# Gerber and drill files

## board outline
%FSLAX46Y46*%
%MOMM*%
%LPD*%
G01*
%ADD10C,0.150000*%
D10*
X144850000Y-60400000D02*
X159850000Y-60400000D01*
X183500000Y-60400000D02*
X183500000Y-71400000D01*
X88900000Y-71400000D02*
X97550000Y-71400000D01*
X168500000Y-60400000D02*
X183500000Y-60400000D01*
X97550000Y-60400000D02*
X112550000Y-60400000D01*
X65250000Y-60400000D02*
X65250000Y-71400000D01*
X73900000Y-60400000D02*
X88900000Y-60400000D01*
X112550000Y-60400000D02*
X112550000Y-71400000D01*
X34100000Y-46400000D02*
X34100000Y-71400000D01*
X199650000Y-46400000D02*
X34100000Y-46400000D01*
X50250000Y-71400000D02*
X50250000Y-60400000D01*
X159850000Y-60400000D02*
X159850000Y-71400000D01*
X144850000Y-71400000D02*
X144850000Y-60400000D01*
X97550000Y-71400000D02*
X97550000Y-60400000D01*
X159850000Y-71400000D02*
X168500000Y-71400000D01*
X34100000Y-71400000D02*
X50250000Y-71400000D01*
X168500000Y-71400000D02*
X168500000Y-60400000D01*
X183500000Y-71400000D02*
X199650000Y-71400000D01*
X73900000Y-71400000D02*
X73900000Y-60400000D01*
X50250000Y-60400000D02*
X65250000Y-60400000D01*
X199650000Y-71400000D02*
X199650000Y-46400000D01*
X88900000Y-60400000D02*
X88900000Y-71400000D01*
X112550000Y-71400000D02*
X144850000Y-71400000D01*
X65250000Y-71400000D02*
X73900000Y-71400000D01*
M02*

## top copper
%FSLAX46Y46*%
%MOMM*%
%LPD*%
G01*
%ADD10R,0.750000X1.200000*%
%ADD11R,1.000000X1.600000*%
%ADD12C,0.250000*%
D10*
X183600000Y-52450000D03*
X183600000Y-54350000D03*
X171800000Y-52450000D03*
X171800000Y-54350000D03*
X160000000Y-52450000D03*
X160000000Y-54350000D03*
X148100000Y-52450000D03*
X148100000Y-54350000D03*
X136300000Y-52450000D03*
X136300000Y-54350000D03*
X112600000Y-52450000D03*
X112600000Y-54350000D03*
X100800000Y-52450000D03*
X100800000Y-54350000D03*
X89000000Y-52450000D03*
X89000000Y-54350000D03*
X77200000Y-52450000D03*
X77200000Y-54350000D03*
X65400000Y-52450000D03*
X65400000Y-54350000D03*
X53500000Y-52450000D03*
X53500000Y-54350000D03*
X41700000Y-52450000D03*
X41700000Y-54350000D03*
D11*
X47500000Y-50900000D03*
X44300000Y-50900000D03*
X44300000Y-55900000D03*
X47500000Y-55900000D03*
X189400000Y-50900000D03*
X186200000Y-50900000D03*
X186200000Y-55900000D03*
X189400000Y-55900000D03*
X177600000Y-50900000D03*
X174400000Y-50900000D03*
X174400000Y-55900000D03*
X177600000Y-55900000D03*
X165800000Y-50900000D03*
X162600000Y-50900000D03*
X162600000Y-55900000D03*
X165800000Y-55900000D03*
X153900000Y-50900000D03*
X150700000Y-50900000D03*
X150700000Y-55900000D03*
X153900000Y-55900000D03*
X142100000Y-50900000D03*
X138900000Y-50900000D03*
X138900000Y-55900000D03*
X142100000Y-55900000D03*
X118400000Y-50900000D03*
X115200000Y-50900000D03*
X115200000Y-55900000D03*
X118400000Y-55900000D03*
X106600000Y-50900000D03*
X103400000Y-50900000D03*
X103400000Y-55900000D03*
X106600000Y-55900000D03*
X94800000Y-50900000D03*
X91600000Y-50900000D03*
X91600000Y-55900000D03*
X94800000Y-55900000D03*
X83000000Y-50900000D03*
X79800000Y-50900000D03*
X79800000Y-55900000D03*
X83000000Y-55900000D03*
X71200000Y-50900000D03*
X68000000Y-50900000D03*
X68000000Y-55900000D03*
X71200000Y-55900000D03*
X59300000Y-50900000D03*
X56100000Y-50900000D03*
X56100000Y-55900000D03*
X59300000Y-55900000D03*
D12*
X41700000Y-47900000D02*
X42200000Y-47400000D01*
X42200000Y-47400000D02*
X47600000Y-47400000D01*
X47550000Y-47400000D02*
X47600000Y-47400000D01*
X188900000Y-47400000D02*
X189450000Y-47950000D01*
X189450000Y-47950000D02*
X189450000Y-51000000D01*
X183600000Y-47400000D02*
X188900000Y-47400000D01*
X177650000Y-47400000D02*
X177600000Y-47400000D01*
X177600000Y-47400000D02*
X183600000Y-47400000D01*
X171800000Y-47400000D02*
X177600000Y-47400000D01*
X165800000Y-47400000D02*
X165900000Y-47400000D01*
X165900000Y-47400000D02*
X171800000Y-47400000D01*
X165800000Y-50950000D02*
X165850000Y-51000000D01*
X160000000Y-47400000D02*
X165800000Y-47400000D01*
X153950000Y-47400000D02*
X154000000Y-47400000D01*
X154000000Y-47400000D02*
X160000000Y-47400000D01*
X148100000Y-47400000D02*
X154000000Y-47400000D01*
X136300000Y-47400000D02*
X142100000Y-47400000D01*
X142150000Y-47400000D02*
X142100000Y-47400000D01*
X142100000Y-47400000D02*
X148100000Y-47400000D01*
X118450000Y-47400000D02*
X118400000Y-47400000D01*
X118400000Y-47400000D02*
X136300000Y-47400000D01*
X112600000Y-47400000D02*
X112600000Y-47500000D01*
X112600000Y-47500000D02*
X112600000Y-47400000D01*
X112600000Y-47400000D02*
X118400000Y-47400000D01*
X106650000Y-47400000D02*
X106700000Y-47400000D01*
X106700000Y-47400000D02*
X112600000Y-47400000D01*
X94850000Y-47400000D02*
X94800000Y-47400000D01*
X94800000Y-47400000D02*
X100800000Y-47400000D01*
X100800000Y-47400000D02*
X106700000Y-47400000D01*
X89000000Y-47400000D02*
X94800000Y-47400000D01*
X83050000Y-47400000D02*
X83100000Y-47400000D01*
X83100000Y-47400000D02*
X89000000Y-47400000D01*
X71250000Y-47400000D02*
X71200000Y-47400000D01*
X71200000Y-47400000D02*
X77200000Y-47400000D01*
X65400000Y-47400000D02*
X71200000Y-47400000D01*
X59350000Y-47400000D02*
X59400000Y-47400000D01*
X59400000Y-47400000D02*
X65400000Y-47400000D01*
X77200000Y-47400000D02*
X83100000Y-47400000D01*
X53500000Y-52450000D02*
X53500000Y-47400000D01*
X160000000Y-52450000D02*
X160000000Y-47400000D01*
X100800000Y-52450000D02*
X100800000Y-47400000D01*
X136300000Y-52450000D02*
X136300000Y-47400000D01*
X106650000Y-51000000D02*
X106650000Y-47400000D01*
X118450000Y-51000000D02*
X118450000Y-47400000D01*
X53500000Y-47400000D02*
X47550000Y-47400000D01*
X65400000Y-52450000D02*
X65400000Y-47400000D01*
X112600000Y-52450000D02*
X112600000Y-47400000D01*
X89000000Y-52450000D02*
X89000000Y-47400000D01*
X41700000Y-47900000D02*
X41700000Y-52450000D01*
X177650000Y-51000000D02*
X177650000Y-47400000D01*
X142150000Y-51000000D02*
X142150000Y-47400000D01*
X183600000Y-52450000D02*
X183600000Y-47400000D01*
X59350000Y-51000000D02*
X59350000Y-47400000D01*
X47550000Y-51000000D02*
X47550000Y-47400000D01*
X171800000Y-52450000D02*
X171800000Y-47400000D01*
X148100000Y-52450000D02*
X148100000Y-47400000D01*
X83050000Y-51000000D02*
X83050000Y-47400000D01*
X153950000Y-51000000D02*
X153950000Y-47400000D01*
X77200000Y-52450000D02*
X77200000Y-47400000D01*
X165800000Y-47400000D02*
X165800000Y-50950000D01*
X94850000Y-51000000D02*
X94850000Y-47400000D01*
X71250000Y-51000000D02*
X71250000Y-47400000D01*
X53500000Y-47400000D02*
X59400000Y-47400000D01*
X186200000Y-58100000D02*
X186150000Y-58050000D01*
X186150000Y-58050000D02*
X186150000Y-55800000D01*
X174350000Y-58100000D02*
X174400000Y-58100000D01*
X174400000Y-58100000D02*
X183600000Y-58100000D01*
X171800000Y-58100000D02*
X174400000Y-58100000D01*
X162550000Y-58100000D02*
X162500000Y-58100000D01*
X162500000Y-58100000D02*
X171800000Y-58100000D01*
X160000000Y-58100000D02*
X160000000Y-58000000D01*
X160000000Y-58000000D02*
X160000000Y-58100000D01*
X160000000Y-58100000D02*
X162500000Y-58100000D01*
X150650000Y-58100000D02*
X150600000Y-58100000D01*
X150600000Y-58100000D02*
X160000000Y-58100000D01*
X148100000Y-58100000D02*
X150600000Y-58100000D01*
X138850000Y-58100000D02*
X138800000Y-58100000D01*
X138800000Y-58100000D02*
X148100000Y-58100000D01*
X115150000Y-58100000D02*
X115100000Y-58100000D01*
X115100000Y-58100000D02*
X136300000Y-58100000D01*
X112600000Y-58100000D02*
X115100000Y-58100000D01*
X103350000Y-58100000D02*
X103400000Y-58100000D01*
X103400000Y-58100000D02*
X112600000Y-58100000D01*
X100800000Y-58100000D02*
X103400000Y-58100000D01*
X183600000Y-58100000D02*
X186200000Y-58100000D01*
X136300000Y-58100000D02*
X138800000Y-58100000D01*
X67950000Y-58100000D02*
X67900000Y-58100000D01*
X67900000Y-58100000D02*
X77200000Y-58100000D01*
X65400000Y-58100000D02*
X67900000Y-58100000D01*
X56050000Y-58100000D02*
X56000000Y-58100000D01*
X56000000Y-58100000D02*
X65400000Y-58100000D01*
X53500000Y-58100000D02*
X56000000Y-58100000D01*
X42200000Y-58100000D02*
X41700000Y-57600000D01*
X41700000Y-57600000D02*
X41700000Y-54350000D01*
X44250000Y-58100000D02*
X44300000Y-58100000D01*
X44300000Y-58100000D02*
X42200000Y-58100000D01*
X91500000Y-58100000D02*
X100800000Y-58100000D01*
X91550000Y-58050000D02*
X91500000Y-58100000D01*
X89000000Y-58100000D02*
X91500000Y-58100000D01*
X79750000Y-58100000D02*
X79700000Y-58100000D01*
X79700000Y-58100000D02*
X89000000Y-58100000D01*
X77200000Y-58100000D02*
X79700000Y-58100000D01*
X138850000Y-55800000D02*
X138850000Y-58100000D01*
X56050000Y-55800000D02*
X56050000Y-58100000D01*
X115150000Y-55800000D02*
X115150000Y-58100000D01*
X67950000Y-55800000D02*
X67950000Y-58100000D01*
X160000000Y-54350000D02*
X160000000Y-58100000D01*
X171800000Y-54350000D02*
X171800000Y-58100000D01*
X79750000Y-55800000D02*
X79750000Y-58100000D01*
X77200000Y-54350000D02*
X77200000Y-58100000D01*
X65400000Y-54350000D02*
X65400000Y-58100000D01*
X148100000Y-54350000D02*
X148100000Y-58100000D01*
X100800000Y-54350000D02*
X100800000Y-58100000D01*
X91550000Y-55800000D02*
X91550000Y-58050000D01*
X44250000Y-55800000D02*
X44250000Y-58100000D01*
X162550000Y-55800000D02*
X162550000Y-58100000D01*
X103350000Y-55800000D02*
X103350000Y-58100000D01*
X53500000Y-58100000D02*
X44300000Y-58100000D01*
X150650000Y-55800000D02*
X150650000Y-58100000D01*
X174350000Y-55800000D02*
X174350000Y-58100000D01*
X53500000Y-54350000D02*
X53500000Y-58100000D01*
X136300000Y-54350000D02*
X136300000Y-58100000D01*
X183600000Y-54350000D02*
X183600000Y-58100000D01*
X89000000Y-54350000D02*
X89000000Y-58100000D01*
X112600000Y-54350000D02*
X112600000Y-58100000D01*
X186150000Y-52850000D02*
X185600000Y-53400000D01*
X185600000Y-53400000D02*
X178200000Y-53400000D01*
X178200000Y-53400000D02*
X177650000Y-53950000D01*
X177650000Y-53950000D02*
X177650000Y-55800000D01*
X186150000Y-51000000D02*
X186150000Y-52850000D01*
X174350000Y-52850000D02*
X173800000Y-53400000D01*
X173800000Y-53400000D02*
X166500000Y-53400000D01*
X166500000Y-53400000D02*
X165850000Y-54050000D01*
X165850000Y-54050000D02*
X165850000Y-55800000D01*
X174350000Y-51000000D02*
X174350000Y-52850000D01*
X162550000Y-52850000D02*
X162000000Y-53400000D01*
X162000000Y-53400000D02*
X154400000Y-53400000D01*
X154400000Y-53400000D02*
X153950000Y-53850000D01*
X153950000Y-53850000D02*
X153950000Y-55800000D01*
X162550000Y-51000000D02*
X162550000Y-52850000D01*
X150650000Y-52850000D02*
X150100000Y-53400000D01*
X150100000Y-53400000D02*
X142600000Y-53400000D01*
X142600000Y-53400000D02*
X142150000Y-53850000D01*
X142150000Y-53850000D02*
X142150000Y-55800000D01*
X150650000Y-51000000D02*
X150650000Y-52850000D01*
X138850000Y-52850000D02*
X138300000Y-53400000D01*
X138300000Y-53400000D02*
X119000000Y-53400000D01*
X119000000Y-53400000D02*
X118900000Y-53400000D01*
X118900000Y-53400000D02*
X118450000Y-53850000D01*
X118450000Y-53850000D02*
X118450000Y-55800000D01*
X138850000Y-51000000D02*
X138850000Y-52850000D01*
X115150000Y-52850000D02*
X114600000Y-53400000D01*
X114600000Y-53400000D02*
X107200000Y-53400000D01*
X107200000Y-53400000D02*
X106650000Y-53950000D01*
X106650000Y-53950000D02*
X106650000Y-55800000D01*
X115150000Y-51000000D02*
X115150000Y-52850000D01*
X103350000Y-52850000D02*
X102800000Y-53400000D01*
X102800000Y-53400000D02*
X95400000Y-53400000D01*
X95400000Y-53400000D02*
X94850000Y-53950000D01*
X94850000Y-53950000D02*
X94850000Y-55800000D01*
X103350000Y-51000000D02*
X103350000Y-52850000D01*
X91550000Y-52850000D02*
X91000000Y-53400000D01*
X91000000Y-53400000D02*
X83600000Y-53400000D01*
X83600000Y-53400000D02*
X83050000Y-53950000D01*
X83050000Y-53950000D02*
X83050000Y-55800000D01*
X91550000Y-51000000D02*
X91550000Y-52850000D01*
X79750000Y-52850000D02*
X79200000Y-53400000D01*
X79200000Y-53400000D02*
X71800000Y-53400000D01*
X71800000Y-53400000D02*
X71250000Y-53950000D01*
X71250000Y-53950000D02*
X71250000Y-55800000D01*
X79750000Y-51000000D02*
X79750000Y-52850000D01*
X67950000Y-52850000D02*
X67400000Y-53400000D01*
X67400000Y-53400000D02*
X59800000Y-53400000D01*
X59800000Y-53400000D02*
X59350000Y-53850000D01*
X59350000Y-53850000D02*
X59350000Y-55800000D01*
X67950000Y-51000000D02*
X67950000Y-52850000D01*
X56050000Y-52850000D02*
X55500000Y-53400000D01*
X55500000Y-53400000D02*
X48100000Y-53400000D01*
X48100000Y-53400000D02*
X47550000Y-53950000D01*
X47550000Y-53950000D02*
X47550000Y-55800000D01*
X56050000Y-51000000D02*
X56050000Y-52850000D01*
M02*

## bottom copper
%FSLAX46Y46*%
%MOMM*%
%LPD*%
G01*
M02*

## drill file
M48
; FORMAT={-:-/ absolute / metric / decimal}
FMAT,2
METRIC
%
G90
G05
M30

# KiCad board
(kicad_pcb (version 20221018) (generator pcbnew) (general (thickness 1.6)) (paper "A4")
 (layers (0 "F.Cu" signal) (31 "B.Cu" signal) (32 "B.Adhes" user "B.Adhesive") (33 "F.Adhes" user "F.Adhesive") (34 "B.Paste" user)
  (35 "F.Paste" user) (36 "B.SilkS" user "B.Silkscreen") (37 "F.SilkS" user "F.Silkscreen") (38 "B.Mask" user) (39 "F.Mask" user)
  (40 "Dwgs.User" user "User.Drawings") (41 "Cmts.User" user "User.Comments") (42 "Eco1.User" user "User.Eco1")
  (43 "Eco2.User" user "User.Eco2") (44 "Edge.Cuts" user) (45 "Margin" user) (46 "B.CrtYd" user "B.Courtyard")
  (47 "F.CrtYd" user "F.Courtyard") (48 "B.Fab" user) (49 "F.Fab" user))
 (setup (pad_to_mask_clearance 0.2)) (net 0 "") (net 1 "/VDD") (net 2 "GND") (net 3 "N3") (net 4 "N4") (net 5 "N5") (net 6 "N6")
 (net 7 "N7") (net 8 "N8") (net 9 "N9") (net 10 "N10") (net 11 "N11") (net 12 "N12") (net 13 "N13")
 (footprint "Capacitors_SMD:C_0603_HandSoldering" (layer "F.Cu") (at 183.6 53.4 -90)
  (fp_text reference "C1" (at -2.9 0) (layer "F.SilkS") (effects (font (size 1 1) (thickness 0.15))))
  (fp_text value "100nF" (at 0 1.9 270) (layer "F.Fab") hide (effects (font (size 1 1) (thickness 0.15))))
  (pad "1" smd rect (at -0.95 0 270) (size 1.2 0.75) (layers "F.Cu" "F.Paste" "F.Mask") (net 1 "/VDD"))
  (pad "2" smd rect (at 0.95 0 270) (size 1.2 0.75) (layers "F.Cu" "F.Paste" "F.Mask") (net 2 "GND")))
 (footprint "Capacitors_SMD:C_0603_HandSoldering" (layer "F.Cu") (at 171.8 53.4 -90)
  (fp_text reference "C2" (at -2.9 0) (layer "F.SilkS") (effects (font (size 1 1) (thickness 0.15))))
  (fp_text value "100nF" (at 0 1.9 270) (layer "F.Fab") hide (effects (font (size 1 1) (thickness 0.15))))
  (pad "1" smd rect (at -0.95 0 270) (size 1.2 0.75) (layers "F.Cu" "F.Paste" "F.Mask") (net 1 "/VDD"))
  (pad "2" smd rect (at 0.95 0 270) (size 1.2 0.75) (layers "F.Cu" "F.Paste" "F.Mask") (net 2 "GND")))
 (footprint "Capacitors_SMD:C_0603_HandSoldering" (layer "F.Cu") (at 160 53.4 -90)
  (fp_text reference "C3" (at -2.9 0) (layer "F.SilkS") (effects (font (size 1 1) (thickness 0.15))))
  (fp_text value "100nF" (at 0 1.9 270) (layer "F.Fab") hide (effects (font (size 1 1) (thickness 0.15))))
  (pad "1" smd rect (at -0.95 0 270) (size 1.2 0.75) (layers "F.Cu" "F.Paste" "F.Mask") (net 1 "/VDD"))
  (pad "2" smd rect (at 0.95 0 270) (size 1.2 0.75) (layers "F.Cu" "F.Paste" "F.Mask") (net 2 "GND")))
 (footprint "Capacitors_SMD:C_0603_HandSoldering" (layer "F.Cu") (at 148.1 53.4 -90)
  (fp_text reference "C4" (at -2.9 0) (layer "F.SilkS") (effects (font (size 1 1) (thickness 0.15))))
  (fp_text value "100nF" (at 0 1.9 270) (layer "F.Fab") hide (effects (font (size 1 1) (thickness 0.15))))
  (pad "1" smd rect (at -0.95 0 270) (size 1.2 0.75) (layers "F.Cu" "F.Paste" "F.Mask") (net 1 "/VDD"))
  (pad "2" smd rect (at 0.95 0 270) (size 1.2 0.75) (layers "F.Cu" "F.Paste" "F.Mask") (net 2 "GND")))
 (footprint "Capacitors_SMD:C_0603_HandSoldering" (layer "F.Cu") (at 136.3 53.4 -90)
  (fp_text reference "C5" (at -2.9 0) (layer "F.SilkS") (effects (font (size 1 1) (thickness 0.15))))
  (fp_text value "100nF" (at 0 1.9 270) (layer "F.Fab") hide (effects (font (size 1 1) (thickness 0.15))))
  (pad "1" smd rect (at -0.95 0 270) (size 1.2 0.75) (layers "F.Cu" "F.Paste" "F.Mask") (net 1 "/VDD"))
  (pad "2" smd rect (at 0.95 0 270) (size 1.2 0.75) (layers "F.Cu" "F.Paste" "F.Mask") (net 2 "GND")))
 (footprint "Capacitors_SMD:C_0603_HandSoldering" (layer "F.Cu") (at 112.6 53.4 -90)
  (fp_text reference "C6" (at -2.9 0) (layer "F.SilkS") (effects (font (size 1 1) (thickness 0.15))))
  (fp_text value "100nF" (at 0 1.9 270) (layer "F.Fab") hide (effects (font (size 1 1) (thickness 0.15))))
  (pad "1" smd rect (at -0.95 0 270) (size 1.2 0.75) (layers "F.Cu" "F.Paste" "F.Mask") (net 1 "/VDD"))
  (pad "2" smd rect (at 0.95 0 270) (size 1.2 0.75) (layers "F.Cu" "F.Paste" "F.Mask") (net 2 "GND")))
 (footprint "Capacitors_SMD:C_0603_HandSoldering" (layer "F.Cu") (at 100.8 53.4 -90)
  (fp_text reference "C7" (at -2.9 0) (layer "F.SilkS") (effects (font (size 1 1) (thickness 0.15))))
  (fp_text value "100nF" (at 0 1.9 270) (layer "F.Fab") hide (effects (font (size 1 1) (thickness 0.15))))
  (pad "1" smd rect (at -0.95 0 270) (size 1.2 0.75) (layers "F.Cu" "F.Paste" "F.Mask") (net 1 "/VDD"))
  (pad "2" smd rect (at 0.95 0 270) (size 1.2 0.75) (layers "F.Cu" "F.Paste" "F.Mask") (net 2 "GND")))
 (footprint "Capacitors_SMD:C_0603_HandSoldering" (layer "F.Cu") (at 89 53.4 -90)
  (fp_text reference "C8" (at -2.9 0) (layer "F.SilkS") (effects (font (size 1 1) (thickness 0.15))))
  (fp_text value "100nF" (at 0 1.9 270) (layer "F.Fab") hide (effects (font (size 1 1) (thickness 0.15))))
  (pad "1" smd rect (at -0.95 0 270) (size 1.2 0.75) (layers "F.Cu" "F.Paste" "F.Mask") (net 1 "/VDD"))
  (pad "2" smd rect (at 0.95 0 270) (size 1.2 0.75) (layers "F.Cu" "F.Paste" "F.Mask") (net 2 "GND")))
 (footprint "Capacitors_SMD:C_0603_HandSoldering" (layer "F.Cu") (at 77.2 53.4 -90)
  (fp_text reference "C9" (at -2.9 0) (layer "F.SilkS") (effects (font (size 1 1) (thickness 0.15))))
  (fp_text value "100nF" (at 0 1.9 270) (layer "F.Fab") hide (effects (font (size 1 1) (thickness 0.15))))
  (pad "1" smd rect (at -0.95 0 270) (size 1.2 0.75) (layers "F.Cu" "F.Paste" "F.Mask") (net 1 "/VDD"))
  (pad "2" smd rect (at 0.95 0 270) (size 1.2 0.75) (layers "F.Cu" "F.Paste" "F.Mask") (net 2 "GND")))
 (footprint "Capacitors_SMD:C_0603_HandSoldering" (layer "F.Cu") (at 65.4 53.4 -90)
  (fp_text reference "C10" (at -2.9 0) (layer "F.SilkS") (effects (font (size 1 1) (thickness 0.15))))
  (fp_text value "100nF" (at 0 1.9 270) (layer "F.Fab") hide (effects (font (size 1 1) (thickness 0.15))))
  (pad "1" smd rect (at -0.95 0 270) (size 1.2 0.75) (layers "F.Cu" "F.Paste" "F.Mask") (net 1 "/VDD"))
  (pad "2" smd rect (at 0.95 0 270) (size 1.2 0.75) (layers "F.Cu" "F.Paste" "F.Mask") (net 2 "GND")))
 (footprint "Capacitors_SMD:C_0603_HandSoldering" (layer "F.Cu") (at 53.5 53.4 -90)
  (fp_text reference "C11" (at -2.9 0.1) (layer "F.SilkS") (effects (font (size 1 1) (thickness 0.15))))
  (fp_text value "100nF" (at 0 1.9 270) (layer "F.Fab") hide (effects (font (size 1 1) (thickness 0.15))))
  (pad "1" smd rect (at -0.95 0 270) (size 1.2 0.75) (layers "F.Cu" "F.Paste" "F.Mask") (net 1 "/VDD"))
  (pad "2" smd rect (at 0.95 0 270) (size 1.2 0.75) (layers "F.Cu" "F.Paste" "F.Mask") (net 2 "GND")))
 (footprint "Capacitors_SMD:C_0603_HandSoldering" (layer "F.Cu") (at 41.7 53.4 -90)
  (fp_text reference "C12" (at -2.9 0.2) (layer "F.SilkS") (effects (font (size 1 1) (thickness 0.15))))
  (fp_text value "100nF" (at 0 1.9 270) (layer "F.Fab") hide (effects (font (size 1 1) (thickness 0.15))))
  (pad "1" smd rect (at -0.95 0 270) (size 1.2 0.75) (layers "F.Cu" "F.Paste" "F.Mask") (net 1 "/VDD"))
  (pad "2" smd rect (at 0.95 0 270) (size 1.2 0.75) (layers "F.Cu" "F.Paste" "F.Mask") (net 2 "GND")))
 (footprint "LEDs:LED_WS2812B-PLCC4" (layer "F.Cu") (at 45.9 53.4 -90)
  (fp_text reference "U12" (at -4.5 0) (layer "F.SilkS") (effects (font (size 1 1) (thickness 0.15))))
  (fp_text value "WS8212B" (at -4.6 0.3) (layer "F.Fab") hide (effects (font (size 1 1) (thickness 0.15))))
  (pad "1" smd rect (at -2.5 -1.6 270) (size 1.6 1) (layers "F.Cu" "F.Paste" "F.Mask") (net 1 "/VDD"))
  (pad "2" smd rect (at -2.5 1.6 270) (size 1.6 1) (layers "F.Cu" "F.Paste" "F.Mask"))
  (pad "3" smd rect (at 2.5 1.6 270) (size 1.6 1) (layers "F.Cu" "F.Paste" "F.Mask") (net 2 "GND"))
  (pad "4" smd rect (at 2.5 -1.6 270) (size 1.6 1) (layers "F.Cu" "F.Paste" "F.Mask") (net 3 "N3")))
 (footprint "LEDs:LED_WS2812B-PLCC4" (layer "F.Cu") (at 187.8 53.4 -90)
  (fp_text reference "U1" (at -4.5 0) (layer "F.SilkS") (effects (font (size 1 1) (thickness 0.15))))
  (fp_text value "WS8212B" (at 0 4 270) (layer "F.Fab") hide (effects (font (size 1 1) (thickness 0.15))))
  (pad "1" smd rect (at -2.5 -1.6 270) (size 1.6 1) (layers "F.Cu" "F.Paste" "F.Mask") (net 1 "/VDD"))
  (pad "2" smd rect (at -2.5 1.6 270) (size 1.6 1) (layers "F.Cu" "F.Paste" "F.Mask") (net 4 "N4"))
  (pad "3" smd rect (at 2.5 1.6 270) (size 1.6 1) (layers "F.Cu" "F.Paste" "F.Mask") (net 2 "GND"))
  (pad "4" smd rect (at 2.5 -1.6 270) (size 1.6 1) (layers "F.Cu" "F.Paste" "F.Mask")))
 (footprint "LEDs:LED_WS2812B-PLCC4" (layer "F.Cu") (at 176 53.4 -90)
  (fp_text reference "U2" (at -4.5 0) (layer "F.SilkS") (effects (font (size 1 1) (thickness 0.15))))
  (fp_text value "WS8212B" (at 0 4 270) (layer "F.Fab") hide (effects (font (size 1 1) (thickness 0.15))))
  (pad "1" smd rect (at -2.5 -1.6 270) (size 1.6 1) (layers "F.Cu" "F.Paste" "F.Mask") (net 1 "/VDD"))
  (pad "2" smd rect (at -2.5 1.6 270) (size 1.6 1) (layers "F.Cu" "F.Paste" "F.Mask") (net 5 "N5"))
  (pad "3" smd rect (at 2.5 1.6 270) (size 1.6 1) (layers "F.Cu" "F.Paste" "F.Mask") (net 2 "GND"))
  (pad "4" smd rect (at 2.5 -1.6 270) (size 1.6 1) (layers "F.Cu" "F.Paste" "F.Mask") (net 4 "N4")))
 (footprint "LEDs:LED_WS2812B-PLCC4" (layer "F.Cu") (at 164.2 53.4 -90)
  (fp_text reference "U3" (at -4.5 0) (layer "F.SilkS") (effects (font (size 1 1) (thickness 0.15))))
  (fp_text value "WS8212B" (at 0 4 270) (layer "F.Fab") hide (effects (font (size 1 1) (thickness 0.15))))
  (pad "1" smd rect (at -2.5 -1.6 270) (size 1.6 1) (layers "F.Cu" "F.Paste" "F.Mask") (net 1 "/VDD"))
  (pad "2" smd rect (at -2.5 1.6 270) (size 1.6 1) (layers "F.Cu" "F.Paste" "F.Mask") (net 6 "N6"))
  (pad "3" smd rect (at 2.5 1.6 270) (size 1.6 1) (layers "F.Cu" "F.Paste" "F.Mask") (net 2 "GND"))
  (pad "4" smd rect (at 2.5 -1.6 270) (size 1.6 1) (layers "F.Cu" "F.Paste" "F.Mask") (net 5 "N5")))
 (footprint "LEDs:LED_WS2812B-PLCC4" (layer "F.Cu") (at 152.3 53.4 -90)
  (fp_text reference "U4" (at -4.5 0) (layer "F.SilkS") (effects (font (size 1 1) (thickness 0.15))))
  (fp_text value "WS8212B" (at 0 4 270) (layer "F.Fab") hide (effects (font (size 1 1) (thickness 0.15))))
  (pad "1" smd rect (at -2.5 -1.6 270) (size 1.6 1) (layers "F.Cu" "F.Paste" "F.Mask") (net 1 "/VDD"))
  (pad "2" smd rect (at -2.5 1.6 270) (size 1.6 1) (layers "F.Cu" "F.Paste" "F.Mask") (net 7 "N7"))
  (pad "3" smd rect (at 2.5 1.6 270) (size 1.6 1) (layers "F.Cu" "F.Paste" "F.Mask") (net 2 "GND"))
  (pad "4" smd rect (at 2.5 -1.6 270) (size 1.6 1) (layers "F.Cu" "F.Paste" "F.Mask") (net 6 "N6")))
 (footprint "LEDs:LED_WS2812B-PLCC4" (layer "F.Cu") (at 140.5 53.4 -90)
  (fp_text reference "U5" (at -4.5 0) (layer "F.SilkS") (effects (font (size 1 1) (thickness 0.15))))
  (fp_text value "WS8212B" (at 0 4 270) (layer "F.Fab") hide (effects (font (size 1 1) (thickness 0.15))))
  (pad "1" smd rect (at -2.5 -1.6 270) (size 1.6 1) (layers "F.Cu" "F.Paste" "F.Mask") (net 1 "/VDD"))
  (pad "2" smd rect (at -2.5 1.6 270) (size 1.6 1) (layers "F.Cu" "F.Paste" "F.Mask") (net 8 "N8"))
  (pad "3" smd rect (at 2.5 1.6 270) (size 1.6 1) (layers "F.Cu" "F.Paste" "F.Mask") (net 2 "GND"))
  (pad "4" smd rect (at 2.5 -1.6 270) (size 1.6 1) (layers "F.Cu" "F.Paste" "F.Mask") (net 7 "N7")))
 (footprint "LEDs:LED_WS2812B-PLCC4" (layer "F.Cu") (at 116.8 53.4 -90)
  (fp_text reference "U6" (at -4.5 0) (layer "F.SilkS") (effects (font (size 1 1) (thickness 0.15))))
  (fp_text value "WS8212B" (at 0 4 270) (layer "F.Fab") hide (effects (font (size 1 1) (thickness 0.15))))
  (pad "1" smd rect (at -2.5 -1.6 270) (size 1.6 1) (layers "F.Cu" "F.Paste" "F.Mask") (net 1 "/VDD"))
  (pad "2" smd rect (at -2.5 1.6 270) (size 1.6 1) (layers "F.Cu" "F.Paste" "F.Mask") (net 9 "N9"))
  (pad "3" smd rect (at 2.5 1.6 270) (size 1.6 1) (layers "F.Cu" "F.Paste" "F.Mask") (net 2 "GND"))
  (pad "4" smd rect (at 2.5 -1.6 270) (size 1.6 1) (layers "F.Cu" "F.Paste" "F.Mask") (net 8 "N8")))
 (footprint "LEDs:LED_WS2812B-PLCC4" (layer "F.Cu") (at 105 53.4 -90)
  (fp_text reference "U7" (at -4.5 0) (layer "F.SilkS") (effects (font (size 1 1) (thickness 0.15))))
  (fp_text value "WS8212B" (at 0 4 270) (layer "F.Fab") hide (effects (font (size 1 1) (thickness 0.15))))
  (pad "1" smd rect (at -2.5 -1.6 270) (size 1.6 1) (layers "F.Cu" "F.Paste" "F.Mask") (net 1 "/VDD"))
  (pad "2" smd rect (at -2.5 1.6 270) (size 1.6 1) (layers "F.Cu" "F.Paste" "F.Mask") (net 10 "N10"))
  (pad "3" smd rect (at 2.5 1.6 270) (size 1.6 1) (layers "F.Cu" "F.Paste" "F.Mask") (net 2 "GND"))
  (pad "4" smd rect (at 2.5 -1.6 270) (size 1.6 1) (layers "F.Cu" "F.Paste" "F.Mask") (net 9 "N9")))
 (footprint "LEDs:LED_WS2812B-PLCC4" (layer "F.Cu") (at 93.2 53.4 -90)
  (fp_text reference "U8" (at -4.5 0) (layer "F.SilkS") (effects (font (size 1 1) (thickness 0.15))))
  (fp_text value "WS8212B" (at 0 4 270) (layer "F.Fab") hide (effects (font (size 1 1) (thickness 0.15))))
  (pad "1" smd rect (at -2.5 -1.6 270) (size 1.6 1) (layers "F.Cu" "F.Paste" "F.Mask") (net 1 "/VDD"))
  (pad "2" smd rect (at -2.5 1.6 270) (size 1.6 1) (layers "F.Cu" "F.Paste" "F.Mask") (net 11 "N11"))
  (pad "3" smd rect (at 2.5 1.6 270) (size 1.6 1) (layers "F.Cu" "F.Paste" "F.Mask") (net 2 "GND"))
  (pad "4" smd rect (at 2.5 -1.6 270) (size 1.6 1) (layers "F.Cu" "F.Paste" "F.Mask") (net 10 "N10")))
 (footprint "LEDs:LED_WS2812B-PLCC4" (layer "F.Cu") (at 81.4 53.4 -90)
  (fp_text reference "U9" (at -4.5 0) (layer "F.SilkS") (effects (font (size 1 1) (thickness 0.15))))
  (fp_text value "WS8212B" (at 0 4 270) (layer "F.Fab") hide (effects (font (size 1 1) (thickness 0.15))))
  (pad "1" smd rect (at -2.5 -1.6 270) (size 1.6 1) (layers "F.Cu" "F.Paste" "F.Mask") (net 1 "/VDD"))
  (pad "2" smd rect (at -2.5 1.6 270) (size 1.6 1) (layers "F.Cu" "F.Paste" "F.Mask") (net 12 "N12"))
  (pad "3" smd rect (at 2.5 1.6 270) (size 1.6 1) (layers "F.Cu" "F.Paste" "F.Mask") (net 2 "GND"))
  (pad "4" smd rect (at 2.5 -1.6 270) (size 1.6 1) (layers "F.Cu" "F.Paste" "F.Mask") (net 11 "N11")))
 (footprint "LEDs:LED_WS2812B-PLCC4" (layer "F.Cu") (at 69.6 53.4 -90)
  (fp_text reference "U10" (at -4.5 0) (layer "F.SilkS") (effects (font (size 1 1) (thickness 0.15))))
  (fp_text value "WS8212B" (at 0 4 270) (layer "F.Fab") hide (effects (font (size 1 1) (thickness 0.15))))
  (pad "1" smd rect (at -2.5 -1.6 270) (size 1.6 1) (layers "F.Cu" "F.Paste" "F.Mask") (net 1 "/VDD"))
  (pad "2" smd rect (at -2.5 1.6 270) (size 1.6 1) (layers "F.Cu" "F.Paste" "F.Mask") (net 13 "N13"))
  (pad "3" smd rect (at 2.5 1.6 270) (size 1.6 1) (layers "F.Cu" "F.Paste" "F.Mask") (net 2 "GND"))
  (pad "4" smd rect (at 2.5 -1.6 270) (size 1.6 1) (layers "F.Cu" "F.Paste" "F.Mask") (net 12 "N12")))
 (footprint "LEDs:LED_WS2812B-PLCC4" (layer "F.Cu") (at 57.7 53.4 -90)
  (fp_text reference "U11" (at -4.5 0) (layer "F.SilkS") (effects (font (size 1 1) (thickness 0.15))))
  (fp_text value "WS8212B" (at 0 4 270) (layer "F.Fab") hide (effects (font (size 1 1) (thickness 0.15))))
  (pad "1" smd rect (at -2.5 -1.6 270) (size 1.6 1) (layers "F.Cu" "F.Paste" "F.Mask") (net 1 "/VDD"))
  (pad "2" smd rect (at -2.5 1.6 270) (size 1.6 1) (layers "F.Cu" "F.Paste" "F.Mask") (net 3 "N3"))
  (pad "3" smd rect (at 2.5 1.6 270) (size 1.6 1) (layers "F.Cu" "F.Paste" "F.Mask") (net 2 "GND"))
  (pad "4" smd rect (at 2.5 -1.6 270) (size 1.6 1) (layers "F.Cu" "F.Paste" "F.Mask") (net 13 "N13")))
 (gr_line (start 144.85 60.4) (end 159.85 60.4) (stroke (width 0.15) (type solid)) (layer "Edge.Cuts"))
 (gr_line (start 183.5 60.4) (end 183.5 71.4) (stroke (width 0.15) (type solid)) (layer "Edge.Cuts"))
 (gr_line (start 88.9 71.4) (end 97.55 71.4) (stroke (width 0.15) (type solid)) (layer "Edge.Cuts"))
 (gr_line (start 168.5 60.4) (end 183.5 60.4) (stroke (width 0.15) (type solid)) (layer "Edge.Cuts"))
 (gr_line (start 97.55 60.4) (end 112.55 60.4) (stroke (width 0.15) (type solid)) (layer "Edge.Cuts"))
 (gr_line (start 65.25 60.4) (end 65.25 71.4) (stroke (width 0.15) (type solid)) (layer "Edge.Cuts"))
 (gr_line (start 73.9 60.4) (end 88.9 60.4) (stroke (width 0.15) (type solid)) (layer "Edge.Cuts"))
 (gr_line (start 112.55 60.4) (end 112.55 71.4) (stroke (width 0.15) (type solid)) (layer "Edge.Cuts"))
 (gr_line (start 34.1 46.4) (end 34.1 71.4) (stroke (width 0.15) (type solid)) (layer "Edge.Cuts"))
 (gr_line (start 199.65 46.4) (end 34.1 46.4) (stroke (width 0.15) (type solid)) (layer "Edge.Cuts"))
 (gr_line (start 50.25 71.4) (end 50.25 60.4) (stroke (width 0.15) (type solid)) (layer "Edge.Cuts"))
 (gr_line (start 159.85 60.4) (end 159.85 71.4) (stroke (width 0.15) (type solid)) (layer "Edge.Cuts"))
 (gr_line (start 144.85 71.4) (end 144.85 60.4) (stroke (width 0.15) (type solid)) (layer "Edge.Cuts"))
 (gr_line (start 97.55 71.4) (end 97.55 60.4) (stroke (width 0.15) (type solid)) (layer "Edge.Cuts"))
 (gr_line (start 159.85 71.4) (end 168.5 71.4) (stroke (width 0.15) (type solid)) (layer "Edge.Cuts"))
 (gr_line (start 34.1 71.4) (end 50.25 71.4) (stroke (width 0.15) (type solid)) (layer "Edge.Cuts"))
 (gr_line (start 168.5 71.4) (end 168.5 60.4) (stroke (width 0.15) (type solid)) (layer "Edge.Cuts"))
 (gr_line (start 183.5 71.4) (end 199.65 71.4) (stroke (width 0.15) (type solid)) (layer "Edge.Cuts"))
 (gr_line (start 73.9 71.4) (end 73.9 60.4) (stroke (width 0.15) (type solid)) (layer "Edge.Cuts"))
 (gr_line (start 50.25 60.4) (end 65.25 60.4) (stroke (width 0.15) (type solid)) (layer "Edge.Cuts"))
 (gr_line (start 199.65 71.4) (end 199.65 46.4) (stroke (width 0.15) (type solid)) (layer "Edge.Cuts"))
 (gr_line (start 88.9 60.4) (end 88.9 71.4) (stroke (width 0.15) (type solid)) (layer "Edge.Cuts"))
 (gr_line (start 112.55 71.4) (end 144.85 71.4) (stroke (width 0.15) (type solid)) (layer "Edge.Cuts"))
 (gr_line (start 65.25 71.4) (end 73.9 71.4) (stroke (width 0.15) (type solid)) (layer "Edge.Cuts"))
 (segment (start 41.7 47.9) (end 42.2 47.4) (width 0.25) (layer "F.Cu") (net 1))
 (segment (start 42.2 47.4) (end 47.6 47.4) (width 0.25) (layer "F.Cu") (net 1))
 (segment (start 47.55 47.4) (end 47.6 47.4) (width 0.25) (layer "F.Cu") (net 1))
 (segment (start 188.9 47.4) (end 189.45 47.95) (width 0.25) (layer "F.Cu") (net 1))
 (segment (start 189.45 47.95) (end 189.45 51) (width 0.25) (layer "F.Cu") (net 1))
 (segment (start 183.6 47.4) (end 188.9 47.4) (width 0.25) (layer "F.Cu") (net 1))
 (segment (start 177.65 47.4) (end 177.6 47.4) (width 0.25) (layer "F.Cu") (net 1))
 (segment (start 177.6 47.4) (end 183.6 47.4) (width 0.25) (layer "F.Cu") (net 1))
 (segment (start 171.8 47.4) (end 177.6 47.4) (width 0.25) (layer "F.Cu") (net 1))
 (segment (start 165.8 47.4) (end 165.9 47.4) (width 0.25) (layer "F.Cu") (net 1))
 (segment (start 165.9 47.4) (end 171.8 47.4) (width 0.25) (layer "F.Cu") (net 1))
 (segment (start 165.8 50.95) (end 165.85 51) (width 0.25) (layer "F.Cu") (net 1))
 (segment (start 160 47.4) (end 165.8 47.4) (width 0.25) (layer "F.Cu") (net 1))
 (segment (start 153.95 47.4) (end 154 47.4) (width 0.25) (layer "F.Cu") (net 1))
 (segment (start 154 47.4) (end 160 47.4) (width 0.25) (layer "F.Cu") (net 1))
 (segment (start 148.1 47.4) (end 154 47.4) (width 0.25) (layer "F.Cu") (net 1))
 (segment (start 136.3 47.4) (end 142.1 47.4) (width 0.25) (layer "F.Cu") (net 1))
 (segment (start 142.15 47.4) (end 142.1 47.4) (width 0.25) (layer "F.Cu") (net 1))
 (segment (start 142.1 47.4) (end 148.1 47.4) (width 0.25) (layer "F.Cu") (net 1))
 (segment (start 118.45 47.4) (end 118.4 47.4) (width 0.25) (layer "F.Cu") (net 1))
 (segment (start 118.4 47.4) (end 136.3 47.4) (width 0.25) (layer "F.Cu") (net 1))
 (segment (start 112.6 47.4) (end 112.6 47.5) (width 0.25) (layer "F.Cu") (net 1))
 (segment (start 112.6 47.5) (end 112.6 47.4) (width 0.25) (layer "F.Cu") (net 1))
 (segment (start 112.6 47.4) (end 118.4 47.4) (width 0.25) (layer "F.Cu") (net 1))
 (segment (start 106.65 47.4) (end 106.7 47.4) (width 0.25) (layer "F.Cu") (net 1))
 (segment (start 106.7 47.4) (end 112.6 47.4) (width 0.25) (layer "F.Cu") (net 1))
 (segment (start 94.85 47.4) (end 94.8 47.4) (width 0.25) (layer "F.Cu") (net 1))
 (segment (start 94.8 47.4) (end 100.8 47.4) (width 0.25) (layer "F.Cu") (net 1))
 (segment (start 100.8 47.4) (end 106.7 47.4) (width 0.25) (layer "F.Cu") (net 1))
 (segment (start 89 47.4) (end 94.8 47.4) (width 0.25) (layer "F.Cu") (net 1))
 (segment (start 83.05 47.4) (end 83.1 47.4) (width 0.25) (layer "F.Cu") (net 1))
 (segment (start 83.1 47.4) (end 89 47.4) (width 0.25) (layer "F.Cu") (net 1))
 (segment (start 71.25 47.4) (end 71.2 47.4) (width 0.25) (layer "F.Cu") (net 1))
 (segment (start 71.2 47.4) (end 77.2 47.4) (width 0.25) (layer "F.Cu") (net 1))
 (segment (start 65.4 47.4) (end 71.2 47.4) (width 0.25) (layer "F.Cu") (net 1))
 (segment (start 59.35 47.4) (end 59.4 47.4) (width 0.25) (layer "F.Cu") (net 1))
 (segment (start 59.4 47.4) (end 65.4 47.4) (width 0.25) (layer "F.Cu") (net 1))
 (segment (start 77.2 47.4) (end 83.1 47.4) (width 0.25) (layer "F.Cu") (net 1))
 (segment (start 53.5 52.45) (end 53.5 47.4) (width 0.25) (layer "F.Cu") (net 1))
 (segment (start 160 52.45) (end 160 47.4) (width 0.25) (layer "F.Cu") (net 1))
 (segment (start 100.8 52.45) (end 100.8 47.4) (width 0.25) (layer "F.Cu") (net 1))
 (segment (start 136.3 52.45) (end 136.3 47.4) (width 0.25) (layer "F.Cu") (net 1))
 (segment (start 106.65 51) (end 106.65 47.4) (width 0.25) (layer "F.Cu") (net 1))
 (segment (start 118.45 51) (end 118.45 47.4) (width 0.25) (layer "F.Cu") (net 1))
 (segment (start 53.5 47.4) (end 47.55 47.4) (width 0.25) (layer "F.Cu") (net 1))
 (segment (start 65.4 52.45) (end 65.4 47.4) (width 0.25) (layer "F.Cu") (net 1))
 (segment (start 112.6 52.45) (end 112.6 47.4) (width 0.25) (layer "F.Cu") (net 1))
 (segment (start 89 52.45) (end 89 47.4) (width 0.25) (layer "F.Cu") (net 1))
 (segment (start 41.7 47.9) (end 41.7 52.45) (width 0.25) (layer "F.Cu") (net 1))
 (segment (start 177.65 51) (end 177.65 47.4) (width 0.25) (layer "F.Cu") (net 1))
 (segment (start 142.15 51) (end 142.15 47.4) (width 0.25) (layer "F.Cu") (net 1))
 (segment (start 183.6 52.45) (end 183.6 47.4) (width 0.25) (layer "F.Cu") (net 1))
 (segment (start 59.35 51) (end 59.35 47.4) (width 0.25) (layer "F.Cu") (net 1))
 (segment (start 47.55 51) (end 47.55 47.4) (width 0.25) (layer "F.Cu") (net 1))
 (segment (start 171.8 52.45) (end 171.8 47.4) (width 0.25) (layer "F.Cu") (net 1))
 (segment (start 148.1 52.45) (end 148.1 47.4) (width 0.25) (layer "F.Cu") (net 1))
 (segment (start 83.05 51) (end 83.05 47.4) (width 0.25) (layer "F.Cu") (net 1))
 (segment (start 153.95 51) (end 153.95 47.4) (width 0.25) (layer "F.Cu") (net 1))
 (segment (start 77.2 52.45) (end 77.2 47.4) (width 0.25) (layer "F.Cu") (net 1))
 (segment (start 165.8 47.4) (end 165.8 50.95) (width 0.25) (layer "F.Cu") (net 1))
 (segment (start 94.85 51) (end 94.85 47.4) (width 0.25) (layer "F.Cu") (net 1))
 (segment (start 71.25 51) (end 71.25 47.4) (width 0.25) (layer "F.Cu") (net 1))
 (segment (start 53.5 47.4) (end 59.4 47.4) (width 0.25) (layer "F.Cu") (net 1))
 (segment (start 186.2 58.1) (end 186.15 58.05) (width 0.25) (layer "F.Cu") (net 2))
 (segment (start 186.15 58.05) (end 186.15 55.8) (width 0.25) (layer "F.Cu") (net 2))
 (segment (start 174.35 58.1) (end 174.4 58.1) (width 0.25) (layer "F.Cu") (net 2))
 (segment (start 174.4 58.1) (end 183.6 58.1) (width 0.25) (layer "F.Cu") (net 2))
 (segment (start 171.8 58.1) (end 174.4 58.1) (width 0.25) (layer "F.Cu") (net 2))
 (segment (start 162.55 58.1) (end 162.5 58.1) (width 0.25) (layer "F.Cu") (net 2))
 (segment (start 162.5 58.1) (end 171.8 58.1) (width 0.25) (layer "F.Cu") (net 2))
 (segment (start 160 58.1) (end 160 58) (width 0.25) (layer "F.Cu") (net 2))
 (segment (start 160 58) (end 160 58.1) (width 0.25) (layer "F.Cu") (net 2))
 (segment (start 160 58.1) (end 162.5 58.1) (width 0.25) (layer "F.Cu") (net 2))
 (segment (start 150.65 58.1) (end 150.6 58.1) (width 0.25) (layer "F.Cu") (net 2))
 (segment (start 150.6 58.1) (end 160 58.1) (width 0.25) (layer "F.Cu") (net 2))
 (segment (start 148.1 58.1) (end 150.6 58.1) (width 0.25) (layer "F.Cu") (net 2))
 (segment (start 138.85 58.1) (end 138.8 58.1) (width 0.25) (layer "F.Cu") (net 2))
 (segment (start 138.8 58.1) (end 148.1 58.1) (width 0.25) (layer "F.Cu") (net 2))
 (segment (start 115.15 58.1) (end 115.1 58.1) (width 0.25) (layer "F.Cu") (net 2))
 (segment (start 115.1 58.1) (end 136.3 58.1) (width 0.25) (layer "F.Cu") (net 2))
 (segment (start 112.6 58.1) (end 115.1 58.1) (width 0.25) (layer "F.Cu") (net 2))
 (segment (start 103.35 58.1) (end 103.4 58.1) (width 0.25) (layer "F.Cu") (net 2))
 (segment (start 103.4 58.1) (end 112.6 58.1) (width 0.25) (layer "F.Cu") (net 2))
 (segment (start 100.8 58.1) (end 103.4 58.1) (width 0.25) (layer "F.Cu") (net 2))
 (segment (start 183.6 58.1) (end 186.2 58.1) (width 0.25) (layer "F.Cu") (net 2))
 (segment (start 136.3 58.1) (end 138.8 58.1) (width 0.25) (layer "F.Cu") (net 2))
 (segment (start 67.95 58.1) (end 67.9 58.1) (width 0.25) (layer "F.Cu") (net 2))
 (segment (start 67.9 58.1) (end 77.2 58.1) (width 0.25) (layer "F.Cu") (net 2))
 (segment (start 65.4 58.1) (end 67.9 58.1) (width 0.25) (layer "F.Cu") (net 2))
 (segment (start 56.05 58.1) (end 56 58.1) (width 0.25) (layer "F.Cu") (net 2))
 (segment (start 56 58.1) (end 65.4 58.1) (width 0.25) (layer "F.Cu") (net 2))
 (segment (start 53.5 58.1) (end 56 58.1) (width 0.25) (layer "F.Cu") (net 2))
 (segment (start 42.2 58.1) (end 41.7 57.6) (width 0.25) (layer "F.Cu") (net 2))
 (segment (start 41.7 57.6) (end 41.7 54.35) (width 0.25) (layer "F.Cu") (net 2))
 (segment (start 44.25 58.1) (end 44.3 58.1) (width 0.25) (layer "F.Cu") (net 2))
 (segment (start 44.3 58.1) (end 42.2 58.1) (width 0.25) (layer "F.Cu") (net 2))
 (segment (start 91.5 58.1) (end 100.8 58.1) (width 0.25) (layer "F.Cu") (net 2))
 (segment (start 91.55 58.05) (end 91.5 58.1) (width 0.25) (layer "F.Cu") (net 2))
 (segment (start 89 58.1) (end 91.5 58.1) (width 0.25) (layer "F.Cu") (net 2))
 (segment (start 79.75 58.1) (end 79.7 58.1) (width 0.25) (layer "F.Cu") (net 2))
 (segment (start 79.7 58.1) (end 89 58.1) (width 0.25) (layer "F.Cu") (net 2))
 (segment (start 77.2 58.1) (end 79.7 58.1) (width 0.25) (layer "F.Cu") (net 2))
 (segment (start 138.85 55.8) (end 138.85 58.1) (width 0.25) (layer "F.Cu") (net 2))
 (segment (start 56.05 55.8) (end 56.05 58.1) (width 0.25) (layer "F.Cu") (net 2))
 (segment (start 115.15 55.8) (end 115.15 58.1) (width 0.25) (layer "F.Cu") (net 2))
 (segment (start 67.95 55.8) (end 67.95 58.1) (width 0.25) (layer "F.Cu") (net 2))
 (segment (start 160 54.35) (end 160 58.1) (width 0.25) (layer "F.Cu") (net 2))
 (segment (start 171.8 54.35) (end 171.8 58.1) (width 0.25) (layer "F.Cu") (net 2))
 (segment (start 79.75 55.8) (end 79.75 58.1) (width 0.25) (layer "F.Cu") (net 2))
 (segment (start 77.2 54.35) (end 77.2 58.1) (width 0.25) (layer "F.Cu") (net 2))
 (segment (start 65.4 54.35) (end 65.4 58.1) (width 0.25) (layer "F.Cu") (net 2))
 (segment (start 148.1 54.35) (end 148.1 58.1) (width 0.25) (layer "F.Cu") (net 2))
 (segment (start 100.8 54.35) (end 100.8 58.1) (width 0.25) (layer "F.Cu") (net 2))
 (segment (start 91.55 55.8) (end 91.55 58.05) (width 0.25) (layer "F.Cu") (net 2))
 (segment (start 44.25 55.8) (end 44.25 58.1) (width 0.25) (layer "F.Cu") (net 2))
 (segment (start 162.55 55.8) (end 162.55 58.1) (width 0.25) (layer "F.Cu") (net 2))
 (segment (start 103.35 55.8) (end 103.35 58.1) (width 0.25) (layer "F.Cu") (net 2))
 (segment (start 53.5 58.1) (end 44.3 58.1) (width 0.25) (layer "F.Cu") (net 2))
 (segment (start 150.65 55.8) (end 150.65 58.1) (width 0.25) (layer "F.Cu") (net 2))
 (segment (start 174.35 55.8) (end 174.35 58.1) (width 0.25) (layer "F.Cu") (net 2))
 (segment (start 53.5 54.35) (end 53.5 58.1) (width 0.25) (layer "F.Cu") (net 2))
 (segment (start 136.3 54.35) (end 136.3 58.1) (width 0.25) (layer "F.Cu") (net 2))
 (segment (start 183.6 54.35) (end 183.6 58.1) (width 0.25) (layer "F.Cu") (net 2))
 (segment (start 89 54.35) (end 89 58.1) (width 0.25) (layer "F.Cu") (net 2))
 (segment (start 112.6 54.35) (end 112.6 58.1) (width 0.25) (layer "F.Cu") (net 2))
 (segment (start 186.15 52.85) (end 185.6 53.4) (width 0.25) (layer "F.Cu") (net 4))
 (segment (start 185.6 53.4) (end 178.2 53.4) (width 0.25) (layer "F.Cu") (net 4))
 (segment (start 178.2 53.4) (end 177.65 53.95) (width 0.25) (layer "F.Cu") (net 4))
 (segment (start 177.65 53.95) (end 177.65 55.8) (width 0.25) (layer "F.Cu") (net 4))
 (segment (start 186.15 51) (end 186.15 52.85) (width 0.25) (layer "F.Cu") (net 4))
 (segment (start 174.35 52.85) (end 173.8 53.4) (width 0.25) (layer "F.Cu") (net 5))
 (segment (start 173.8 53.4) (end 166.5 53.4) (width 0.25) (layer "F.Cu") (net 5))
 (segment (start 166.5 53.4) (end 165.85 54.05) (width 0.25) (layer "F.Cu") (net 5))
 (segment (start 165.85 54.05) (end 165.85 55.8) (width 0.25) (layer "F.Cu") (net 5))
 (segment (start 174.35 51) (end 174.35 52.85) (width 0.25) (layer "F.Cu") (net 5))
 (segment (start 162.55 52.85) (end 162 53.4) (width 0.25) (layer "F.Cu") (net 6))
 (segment (start 162 53.4) (end 154.4 53.4) (width 0.25) (layer "F.Cu") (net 6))
 (segment (start 154.4 53.4) (end 153.95 53.85) (width 0.25) (layer "F.Cu") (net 6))
 (segment (start 153.95 53.85) (end 153.95 55.8) (width 0.25) (layer "F.Cu") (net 6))
 (segment (start 162.55 51) (end 162.55 52.85) (width 0.25) (layer "F.Cu") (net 6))
 (segment (start 150.65 52.85) (end 150.1 53.4) (width 0.25) (layer "F.Cu") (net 7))
 (segment (start 150.1 53.4) (end 142.6 53.4) (width 0.25) (layer "F.Cu") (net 7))
 (segment (start 142.6 53.4) (end 142.15 53.85) (width 0.25) (layer "F.Cu") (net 7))
 (segment (start 142.15 53.85) (end 142.15 55.8) (width 0.25) (layer "F.Cu") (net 7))
 (segment (start 150.65 51) (end 150.65 52.85) (width 0.25) (layer "F.Cu") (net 7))
 (segment (start 138.85 52.85) (end 138.3 53.4) (width 0.25) (layer "F.Cu") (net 8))
 (segment (start 138.3 53.4) (end 119 53.4) (width 0.25) (layer "F.Cu") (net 8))
 (segment (start 119 53.4) (end 118.9 53.4) (width 0.25) (layer "F.Cu") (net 8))
 (segment (start 118.9 53.4) (end 118.45 53.85) (width 0.25) (layer "F.Cu") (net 8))
 (segment (start 118.45 53.85) (end 118.45 55.8) (width 0.25) (layer "F.Cu") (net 8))
 (segment (start 138.85 51) (end 138.85 52.85) (width 0.25) (layer "F.Cu") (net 8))
 (segment (start 115.15 52.85) (end 114.6 53.4) (width 0.25) (layer "F.Cu") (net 9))
 (segment (start 114.6 53.4) (end 107.2 53.4) (width 0.25) (layer "F.Cu") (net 9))
 (segment (start 107.2 53.4) (end 106.65 53.95) (width 0.25) (layer "F.Cu") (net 9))
 (segment (start 106.65 53.95) (end 106.65 55.8) (width 0.25) (layer "F.Cu") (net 9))
 (segment (start 115.15 51) (end 115.15 52.85) (width 0.25) (layer "F.Cu") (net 9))
 (segment (start 103.35 52.85) (end 102.8 53.4) (width 0.25) (layer "F.Cu") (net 10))
 (segment (start 102.8 53.4) (end 95.4 53.4) (width 0.25) (layer "F.Cu") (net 10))
 (segment (start 95.4 53.4) (end 94.85 53.95) (width 0.25) (layer "F.Cu") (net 10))
 (segment (start 94.85 53.95) (end 94.85 55.8) (width 0.25) (layer "F.Cu") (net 10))
 (segment (start 103.35 51) (end 103.35 52.85) (width 0.25) (layer "F.Cu") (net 10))
 (segment (start 91.55 52.85) (end 91 53.4) (width 0.25) (layer "F.Cu") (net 11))
 (segment (start 91 53.4) (end 83.6 53.4) (width 0.25) (layer "F.Cu") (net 11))
 (segment (start 83.6 53.4) (end 83.05 53.95) (width 0.25) (layer "F.Cu") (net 11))
 (segment (start 83.05 53.95) (end 83.05 55.8) (width 0.25) (layer "F.Cu") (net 11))
 (segment (start 91.55 51) (end 91.55 52.85) (width 0.25) (layer "F.Cu") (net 11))
 (segment (start 79.75 52.85) (end 79.2 53.4) (width 0.25) (layer "F.Cu") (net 12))
 (segment (start 79.2 53.4) (end 71.8 53.4) (width 0.25) (layer "F.Cu") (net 12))
 (segment (start 71.8 53.4) (end 71.25 53.95) (width 0.25) (layer "F.Cu") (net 12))
 (segment (start 71.25 53.95) (end 71.25 55.8) (width 0.25) (layer "F.Cu") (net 12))
 (segment (start 79.75 51) (end 79.75 52.85) (width 0.25) (layer "F.Cu") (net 12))
 (segment (start 67.95 52.85) (end 67.4 53.4) (width 0.25) (layer "F.Cu") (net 13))
 (segment (start 67.4 53.4) (end 59.8 53.4) (width 0.25) (layer "F.Cu") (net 13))
 (segment (start 59.8 53.4) (end 59.35 53.85) (width 0.25) (layer "F.Cu") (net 13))
 (segment (start 59.35 53.85) (end 59.35 55.8) (width 0.25) (layer "F.Cu") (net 13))
 (segment (start 67.95 51) (end 67.95 52.85) (width 0.25) (layer "F.Cu") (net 13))
 (segment (start 56.05 52.85) (end 55.5 53.4) (width 0.25) (layer "F.Cu") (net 3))
 (segment (start 55.5 53.4) (end 48.1 53.4) (width 0.25) (layer "F.Cu") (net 3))
 (segment (start 48.1 53.4) (end 47.55 53.95) (width 0.25) (layer "F.Cu") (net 3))
 (segment (start 47.55 53.95) (end 47.55 55.8) (width 0.25) (layer "F.Cu") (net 3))
 (segment (start 56.05 51) (end 56.05 52.85) (width 0.25) (layer "F.Cu") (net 3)))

